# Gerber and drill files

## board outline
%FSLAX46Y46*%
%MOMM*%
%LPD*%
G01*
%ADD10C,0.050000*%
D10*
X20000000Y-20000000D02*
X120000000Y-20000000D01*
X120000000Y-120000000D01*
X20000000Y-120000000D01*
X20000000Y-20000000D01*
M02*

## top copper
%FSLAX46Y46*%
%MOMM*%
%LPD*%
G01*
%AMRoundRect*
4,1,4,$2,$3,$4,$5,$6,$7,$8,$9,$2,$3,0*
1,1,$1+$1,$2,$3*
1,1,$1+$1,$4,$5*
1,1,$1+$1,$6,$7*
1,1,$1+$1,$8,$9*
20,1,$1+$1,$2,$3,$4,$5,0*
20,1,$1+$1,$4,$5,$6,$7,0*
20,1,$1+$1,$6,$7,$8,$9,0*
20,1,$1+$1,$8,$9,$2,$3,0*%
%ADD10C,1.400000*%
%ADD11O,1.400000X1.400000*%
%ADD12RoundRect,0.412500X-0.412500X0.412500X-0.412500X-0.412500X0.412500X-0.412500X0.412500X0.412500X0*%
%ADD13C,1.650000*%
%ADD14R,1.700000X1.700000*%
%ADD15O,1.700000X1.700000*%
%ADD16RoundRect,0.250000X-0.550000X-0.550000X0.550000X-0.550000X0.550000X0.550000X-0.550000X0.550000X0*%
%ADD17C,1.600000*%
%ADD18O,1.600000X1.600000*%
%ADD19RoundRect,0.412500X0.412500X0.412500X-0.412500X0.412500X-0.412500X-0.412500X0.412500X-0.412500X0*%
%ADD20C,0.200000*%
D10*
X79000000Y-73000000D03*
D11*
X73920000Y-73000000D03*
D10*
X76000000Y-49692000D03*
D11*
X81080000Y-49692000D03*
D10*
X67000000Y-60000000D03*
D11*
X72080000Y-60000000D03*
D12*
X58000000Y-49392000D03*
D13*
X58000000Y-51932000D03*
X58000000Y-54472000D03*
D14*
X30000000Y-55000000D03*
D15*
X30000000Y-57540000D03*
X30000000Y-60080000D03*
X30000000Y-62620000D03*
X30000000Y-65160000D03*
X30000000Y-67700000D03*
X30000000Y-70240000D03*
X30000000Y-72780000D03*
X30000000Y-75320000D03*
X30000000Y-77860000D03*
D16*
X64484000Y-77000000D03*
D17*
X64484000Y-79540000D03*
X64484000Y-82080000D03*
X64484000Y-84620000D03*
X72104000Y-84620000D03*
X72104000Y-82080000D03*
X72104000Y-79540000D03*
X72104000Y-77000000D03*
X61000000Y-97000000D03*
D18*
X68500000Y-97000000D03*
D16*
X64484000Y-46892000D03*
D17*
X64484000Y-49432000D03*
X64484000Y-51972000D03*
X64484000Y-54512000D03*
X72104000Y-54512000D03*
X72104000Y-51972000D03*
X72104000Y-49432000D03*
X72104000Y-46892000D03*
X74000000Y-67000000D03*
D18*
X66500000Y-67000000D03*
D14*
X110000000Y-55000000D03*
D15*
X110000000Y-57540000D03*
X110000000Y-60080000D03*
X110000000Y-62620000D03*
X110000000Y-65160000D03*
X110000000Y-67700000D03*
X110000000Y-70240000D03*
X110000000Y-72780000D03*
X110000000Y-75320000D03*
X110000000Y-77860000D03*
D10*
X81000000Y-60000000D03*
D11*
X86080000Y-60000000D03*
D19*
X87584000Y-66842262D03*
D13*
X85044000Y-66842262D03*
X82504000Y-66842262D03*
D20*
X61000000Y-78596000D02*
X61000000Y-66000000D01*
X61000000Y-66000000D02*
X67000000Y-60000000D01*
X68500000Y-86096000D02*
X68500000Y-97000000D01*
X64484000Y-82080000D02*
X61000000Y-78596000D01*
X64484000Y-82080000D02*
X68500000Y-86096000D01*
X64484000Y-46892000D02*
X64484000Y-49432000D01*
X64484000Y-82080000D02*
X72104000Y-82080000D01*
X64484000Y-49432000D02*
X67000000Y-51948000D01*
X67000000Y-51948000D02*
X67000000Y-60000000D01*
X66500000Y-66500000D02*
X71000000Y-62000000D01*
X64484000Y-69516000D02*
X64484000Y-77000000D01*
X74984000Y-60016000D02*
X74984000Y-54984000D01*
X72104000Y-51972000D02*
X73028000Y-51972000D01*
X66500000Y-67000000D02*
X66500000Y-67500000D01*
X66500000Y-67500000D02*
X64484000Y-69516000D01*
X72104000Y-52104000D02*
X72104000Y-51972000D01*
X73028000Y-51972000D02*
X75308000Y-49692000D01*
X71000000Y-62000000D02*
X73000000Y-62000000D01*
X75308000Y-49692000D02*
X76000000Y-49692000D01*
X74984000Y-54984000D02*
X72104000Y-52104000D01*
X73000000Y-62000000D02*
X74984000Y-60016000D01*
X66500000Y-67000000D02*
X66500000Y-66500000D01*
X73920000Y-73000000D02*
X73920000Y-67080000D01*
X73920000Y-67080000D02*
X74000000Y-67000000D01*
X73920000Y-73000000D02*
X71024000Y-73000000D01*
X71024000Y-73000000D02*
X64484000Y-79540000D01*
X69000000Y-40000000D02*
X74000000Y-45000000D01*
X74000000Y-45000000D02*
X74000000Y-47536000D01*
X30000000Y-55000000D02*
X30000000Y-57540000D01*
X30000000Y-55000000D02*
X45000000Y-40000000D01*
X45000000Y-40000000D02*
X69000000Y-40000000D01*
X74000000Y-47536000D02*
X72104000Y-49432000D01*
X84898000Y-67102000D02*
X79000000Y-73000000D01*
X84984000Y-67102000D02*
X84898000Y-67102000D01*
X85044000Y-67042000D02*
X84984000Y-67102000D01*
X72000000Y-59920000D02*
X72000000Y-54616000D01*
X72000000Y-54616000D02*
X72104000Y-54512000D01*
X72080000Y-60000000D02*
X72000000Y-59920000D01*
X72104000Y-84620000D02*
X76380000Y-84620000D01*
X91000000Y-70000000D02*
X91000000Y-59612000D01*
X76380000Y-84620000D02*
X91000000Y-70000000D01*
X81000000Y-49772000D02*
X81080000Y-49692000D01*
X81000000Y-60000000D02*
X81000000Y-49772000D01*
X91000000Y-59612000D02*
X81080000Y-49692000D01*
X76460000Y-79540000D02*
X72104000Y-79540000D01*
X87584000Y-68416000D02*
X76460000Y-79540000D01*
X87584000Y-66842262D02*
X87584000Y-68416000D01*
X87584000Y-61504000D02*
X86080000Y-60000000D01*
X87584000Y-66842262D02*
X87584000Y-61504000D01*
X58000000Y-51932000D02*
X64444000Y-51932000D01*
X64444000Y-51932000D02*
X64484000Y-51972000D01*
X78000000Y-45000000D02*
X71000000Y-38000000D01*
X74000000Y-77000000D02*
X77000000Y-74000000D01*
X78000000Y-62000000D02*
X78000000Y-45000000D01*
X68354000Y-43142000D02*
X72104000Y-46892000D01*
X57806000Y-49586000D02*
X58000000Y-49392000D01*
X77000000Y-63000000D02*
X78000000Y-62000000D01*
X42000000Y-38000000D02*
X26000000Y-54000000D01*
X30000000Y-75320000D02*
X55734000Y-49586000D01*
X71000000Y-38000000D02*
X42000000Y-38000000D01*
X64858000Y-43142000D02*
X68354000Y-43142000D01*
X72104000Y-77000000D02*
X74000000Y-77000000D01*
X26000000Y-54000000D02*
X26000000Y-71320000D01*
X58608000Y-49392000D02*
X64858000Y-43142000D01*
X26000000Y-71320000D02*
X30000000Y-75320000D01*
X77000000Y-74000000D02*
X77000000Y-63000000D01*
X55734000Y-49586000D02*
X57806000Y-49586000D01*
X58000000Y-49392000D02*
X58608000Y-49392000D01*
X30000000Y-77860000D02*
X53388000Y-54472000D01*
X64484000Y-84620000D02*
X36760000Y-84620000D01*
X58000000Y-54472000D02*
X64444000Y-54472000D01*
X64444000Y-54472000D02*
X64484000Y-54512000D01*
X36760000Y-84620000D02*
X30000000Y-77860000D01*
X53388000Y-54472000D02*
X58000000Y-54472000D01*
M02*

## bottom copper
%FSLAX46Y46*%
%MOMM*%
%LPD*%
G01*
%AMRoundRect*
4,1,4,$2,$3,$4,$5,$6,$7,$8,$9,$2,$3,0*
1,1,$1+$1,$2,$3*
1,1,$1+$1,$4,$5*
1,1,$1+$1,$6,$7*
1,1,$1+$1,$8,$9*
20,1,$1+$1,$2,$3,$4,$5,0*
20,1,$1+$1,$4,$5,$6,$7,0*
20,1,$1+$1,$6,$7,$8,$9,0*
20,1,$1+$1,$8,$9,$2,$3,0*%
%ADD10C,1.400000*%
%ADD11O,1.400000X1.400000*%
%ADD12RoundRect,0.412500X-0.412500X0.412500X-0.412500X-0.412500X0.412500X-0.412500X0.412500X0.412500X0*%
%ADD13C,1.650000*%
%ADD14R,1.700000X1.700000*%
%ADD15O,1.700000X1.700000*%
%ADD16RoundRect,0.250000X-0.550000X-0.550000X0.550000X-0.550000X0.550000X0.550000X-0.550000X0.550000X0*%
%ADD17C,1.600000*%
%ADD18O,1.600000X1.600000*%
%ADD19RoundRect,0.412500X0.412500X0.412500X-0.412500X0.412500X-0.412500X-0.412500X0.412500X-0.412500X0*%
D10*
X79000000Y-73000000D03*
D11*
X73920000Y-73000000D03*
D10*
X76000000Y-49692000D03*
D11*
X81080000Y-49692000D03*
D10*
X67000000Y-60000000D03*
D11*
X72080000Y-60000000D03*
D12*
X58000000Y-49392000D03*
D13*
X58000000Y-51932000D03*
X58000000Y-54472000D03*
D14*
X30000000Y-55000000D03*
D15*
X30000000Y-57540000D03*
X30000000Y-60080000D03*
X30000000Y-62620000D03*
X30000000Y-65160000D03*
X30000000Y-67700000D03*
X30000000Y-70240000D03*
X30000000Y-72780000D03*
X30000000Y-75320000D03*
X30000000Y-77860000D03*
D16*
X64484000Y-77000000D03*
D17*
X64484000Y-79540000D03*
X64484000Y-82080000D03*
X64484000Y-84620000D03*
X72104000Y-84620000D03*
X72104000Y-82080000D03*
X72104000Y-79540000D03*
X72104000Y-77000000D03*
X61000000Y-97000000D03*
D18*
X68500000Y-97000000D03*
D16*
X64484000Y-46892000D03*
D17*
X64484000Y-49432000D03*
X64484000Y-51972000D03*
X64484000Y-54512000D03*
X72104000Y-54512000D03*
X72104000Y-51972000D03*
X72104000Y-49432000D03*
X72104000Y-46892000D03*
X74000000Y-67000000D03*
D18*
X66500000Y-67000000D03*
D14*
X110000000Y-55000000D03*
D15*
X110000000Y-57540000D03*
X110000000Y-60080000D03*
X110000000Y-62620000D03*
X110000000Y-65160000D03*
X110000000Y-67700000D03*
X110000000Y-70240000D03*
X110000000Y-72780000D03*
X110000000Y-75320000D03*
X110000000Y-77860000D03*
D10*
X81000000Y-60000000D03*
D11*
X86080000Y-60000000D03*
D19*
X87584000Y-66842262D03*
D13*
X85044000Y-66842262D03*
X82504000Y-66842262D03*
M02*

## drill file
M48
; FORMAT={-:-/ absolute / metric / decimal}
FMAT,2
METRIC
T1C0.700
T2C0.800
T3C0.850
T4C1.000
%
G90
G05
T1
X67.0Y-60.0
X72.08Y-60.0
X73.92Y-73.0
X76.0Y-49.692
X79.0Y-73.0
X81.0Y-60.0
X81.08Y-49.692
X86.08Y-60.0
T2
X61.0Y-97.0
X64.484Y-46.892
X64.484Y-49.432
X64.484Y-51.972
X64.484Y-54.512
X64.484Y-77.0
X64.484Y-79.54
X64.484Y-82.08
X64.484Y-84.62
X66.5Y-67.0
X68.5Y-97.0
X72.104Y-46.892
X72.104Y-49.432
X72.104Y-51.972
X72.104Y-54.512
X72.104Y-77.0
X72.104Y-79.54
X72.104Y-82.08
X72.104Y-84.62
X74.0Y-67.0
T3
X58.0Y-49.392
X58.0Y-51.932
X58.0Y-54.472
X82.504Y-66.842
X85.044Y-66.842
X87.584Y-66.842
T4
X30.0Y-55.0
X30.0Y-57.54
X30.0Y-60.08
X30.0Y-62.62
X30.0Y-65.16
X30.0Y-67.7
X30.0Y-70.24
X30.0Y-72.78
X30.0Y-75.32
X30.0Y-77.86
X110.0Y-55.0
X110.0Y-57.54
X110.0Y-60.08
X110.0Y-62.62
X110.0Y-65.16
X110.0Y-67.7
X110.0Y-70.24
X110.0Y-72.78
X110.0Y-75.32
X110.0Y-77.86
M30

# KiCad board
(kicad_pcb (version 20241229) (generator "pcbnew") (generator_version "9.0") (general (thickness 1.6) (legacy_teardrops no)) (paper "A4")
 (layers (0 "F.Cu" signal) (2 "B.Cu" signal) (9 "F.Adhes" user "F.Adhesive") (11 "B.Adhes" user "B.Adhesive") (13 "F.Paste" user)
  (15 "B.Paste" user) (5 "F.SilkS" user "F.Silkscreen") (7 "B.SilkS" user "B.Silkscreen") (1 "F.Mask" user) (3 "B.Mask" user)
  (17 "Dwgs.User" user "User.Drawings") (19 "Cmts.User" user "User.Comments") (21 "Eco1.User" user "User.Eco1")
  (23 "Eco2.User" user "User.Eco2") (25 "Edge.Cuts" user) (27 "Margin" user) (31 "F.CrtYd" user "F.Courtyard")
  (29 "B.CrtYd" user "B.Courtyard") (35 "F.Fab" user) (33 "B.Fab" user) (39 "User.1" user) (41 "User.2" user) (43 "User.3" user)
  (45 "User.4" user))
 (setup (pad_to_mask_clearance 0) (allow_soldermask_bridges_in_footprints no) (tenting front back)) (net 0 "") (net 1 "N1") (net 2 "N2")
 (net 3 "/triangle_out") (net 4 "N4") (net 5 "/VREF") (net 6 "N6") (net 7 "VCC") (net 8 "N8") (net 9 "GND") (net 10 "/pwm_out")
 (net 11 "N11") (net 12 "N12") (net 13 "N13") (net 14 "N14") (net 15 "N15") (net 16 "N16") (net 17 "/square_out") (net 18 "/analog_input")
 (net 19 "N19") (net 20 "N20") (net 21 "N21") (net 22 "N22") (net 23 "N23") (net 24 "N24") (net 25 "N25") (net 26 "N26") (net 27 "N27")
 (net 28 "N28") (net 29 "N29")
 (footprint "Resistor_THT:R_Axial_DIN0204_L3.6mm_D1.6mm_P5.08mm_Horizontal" (layer "F.Cu") (at 79 73 180)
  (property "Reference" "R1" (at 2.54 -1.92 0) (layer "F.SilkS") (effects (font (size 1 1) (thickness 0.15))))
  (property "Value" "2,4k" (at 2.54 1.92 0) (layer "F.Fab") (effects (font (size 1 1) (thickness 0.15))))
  (pad "1" thru_hole circle (at 0 0 180) (size 1.4 1.4) (drill 0.7) (layers "*.Cu" "*.Mask") (remove_unused_layers no) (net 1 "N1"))
  (pad "2" thru_hole oval (at 5.08 0 180) (size 1.4 1.4) (drill 0.7) (layers "*.Cu" "*.Mask") (remove_unused_layers no) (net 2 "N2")))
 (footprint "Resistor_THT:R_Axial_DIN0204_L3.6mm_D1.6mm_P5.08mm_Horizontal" (layer "F.Cu") (at 76 49.692)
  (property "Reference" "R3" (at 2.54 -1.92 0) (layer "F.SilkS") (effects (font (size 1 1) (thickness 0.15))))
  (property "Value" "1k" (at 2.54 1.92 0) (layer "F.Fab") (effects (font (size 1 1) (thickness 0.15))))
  (pad "1" thru_hole circle (at 0 0) (size 1.4 1.4) (drill 0.7) (layers "*.Cu" "*.Mask") (remove_unused_layers no) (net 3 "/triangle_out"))
  (pad "2" thru_hole oval (at 5.08 0) (size 1.4 1.4) (drill 0.7) (layers "*.Cu" "*.Mask") (remove_unused_layers no) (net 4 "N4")))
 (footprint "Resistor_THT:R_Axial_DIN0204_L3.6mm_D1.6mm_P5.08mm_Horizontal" (layer "F.Cu") (at 67 60)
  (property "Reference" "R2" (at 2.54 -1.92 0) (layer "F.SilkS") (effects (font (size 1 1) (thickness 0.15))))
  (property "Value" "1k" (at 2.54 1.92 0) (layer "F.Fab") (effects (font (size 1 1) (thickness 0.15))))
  (pad "1" thru_hole circle (at 0 0) (size 1.4 1.4) (drill 0.7) (layers "*.Cu" "*.Mask") (remove_unused_layers no) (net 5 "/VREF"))
  (pad "2" thru_hole oval (at 5.08 0) (size 1.4 1.4) (drill 0.7) (layers "*.Cu" "*.Mask") (remove_unused_layers no) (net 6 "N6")))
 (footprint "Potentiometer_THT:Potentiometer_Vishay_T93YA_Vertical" (layer "F.Cu") (at 58 49.392 -90)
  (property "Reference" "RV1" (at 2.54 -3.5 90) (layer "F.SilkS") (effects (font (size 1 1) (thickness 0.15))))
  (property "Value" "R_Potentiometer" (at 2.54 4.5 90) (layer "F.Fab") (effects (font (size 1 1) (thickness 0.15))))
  (pad "1" thru_hole roundrect (at 0 0 270) (size 1.65 1.65) (drill 0.85) (layers "*.Cu" "*.Mask") (remove_unused_layers no)
   (roundrect_rratio 0.25) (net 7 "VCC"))
  (pad "2" thru_hole circle (at 2.54 0 270) (size 1.65 1.65) (drill 0.85) (layers "*.Cu" "*.Mask") (remove_unused_layers no) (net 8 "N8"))
  (pad "3" thru_hole circle (at 5.08 0 270) (size 1.65 1.65) (drill 0.85) (layers "*.Cu" "*.Mask") (remove_unused_layers no) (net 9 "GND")))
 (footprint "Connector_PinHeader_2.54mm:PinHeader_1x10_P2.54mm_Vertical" (layer "F.Cu") (at 30 55)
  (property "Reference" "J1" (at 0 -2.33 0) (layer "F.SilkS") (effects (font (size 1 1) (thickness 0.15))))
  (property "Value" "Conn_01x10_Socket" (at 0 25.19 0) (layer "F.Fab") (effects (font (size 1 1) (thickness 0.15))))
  (pad "1" thru_hole rect (at 0 0) (size 1.7 1.7) (drill 1) (layers "*.Cu" "*.Mask") (remove_unused_layers no) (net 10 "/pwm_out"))
  (pad "2" thru_hole oval (at 0 2.54) (size 1.7 1.7) (drill 1) (layers "*.Cu" "*.Mask") (remove_unused_layers no) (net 10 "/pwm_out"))
  (pad "3" thru_hole oval (at 0 5.08) (size 1.7 1.7) (drill 1) (layers "*.Cu" "*.Mask") (remove_unused_layers no) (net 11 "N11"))
  (pad "4" thru_hole oval (at 0 7.62) (size 1.7 1.7) (drill 1) (layers "*.Cu" "*.Mask") (remove_unused_layers no) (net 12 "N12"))
  (pad "5" thru_hole oval (at 0 10.16) (size 1.7 1.7) (drill 1) (layers "*.Cu" "*.Mask") (remove_unused_layers no) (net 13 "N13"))
  (pad "6" thru_hole oval (at 0 12.7) (size 1.7 1.7) (drill 1) (layers "*.Cu" "*.Mask") (remove_unused_layers no) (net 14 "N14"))
  (pad "7" thru_hole oval (at 0 15.24) (size 1.7 1.7) (drill 1) (layers "*.Cu" "*.Mask") (remove_unused_layers no) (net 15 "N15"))
  (pad "8" thru_hole oval (at 0 17.78) (size 1.7 1.7) (drill 1) (layers "*.Cu" "*.Mask") (remove_unused_layers no) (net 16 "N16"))
  (pad "9" thru_hole oval (at 0 20.32) (size 1.7 1.7) (drill 1) (layers "*.Cu" "*.Mask") (remove_unused_layers no) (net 7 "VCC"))
  (pad "10" thru_hole oval (at 0 22.86) (size 1.7 1.7) (drill 1) (layers "*.Cu" "*.Mask") (remove_unused_layers no) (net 9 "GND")))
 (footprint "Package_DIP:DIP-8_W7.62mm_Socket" (layer "F.Cu") (at 64.484 77)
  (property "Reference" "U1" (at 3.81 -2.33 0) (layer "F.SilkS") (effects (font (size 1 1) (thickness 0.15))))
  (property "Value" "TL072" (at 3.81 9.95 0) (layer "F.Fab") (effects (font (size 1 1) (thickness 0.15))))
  (pad "1" thru_hole roundrect (at 0 0) (size 1.6 1.6) (drill 0.8) (layers "*.Cu" "*.Mask") (remove_unused_layers no)
   (roundrect_rratio 0.15625) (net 3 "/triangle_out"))
  (pad "2" thru_hole circle (at 0 2.54) (size 1.6 1.6) (drill 0.8) (layers "*.Cu" "*.Mask") (remove_unused_layers no) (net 2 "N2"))
  (pad "3" thru_hole circle (at 0 5.08) (size 1.6 1.6) (drill 0.8) (layers "*.Cu" "*.Mask") (remove_unused_layers no) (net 5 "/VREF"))
  (pad "4" thru_hole circle (at 0 7.62) (size 1.6 1.6) (drill 0.8) (layers "*.Cu" "*.Mask") (remove_unused_layers no) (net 9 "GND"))
  (pad "5" thru_hole circle (at 7.62 7.62) (size 1.6 1.6) (drill 0.8) (layers "*.Cu" "*.Mask") (remove_unused_layers no) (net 4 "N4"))
  (pad "6" thru_hole circle (at 7.62 5.08) (size 1.6 1.6) (drill 0.8) (layers "*.Cu" "*.Mask") (remove_unused_layers no) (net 5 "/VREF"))
  (pad "7" thru_hole circle (at 7.62 2.54) (size 1.6 1.6) (drill 0.8) (layers "*.Cu" "*.Mask") (remove_unused_layers no)
   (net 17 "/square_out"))
  (pad "8" thru_hole circle (at 7.62 0) (size 1.6 1.6) (drill 0.8) (layers "*.Cu" "*.Mask") (remove_unused_layers no) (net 7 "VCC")))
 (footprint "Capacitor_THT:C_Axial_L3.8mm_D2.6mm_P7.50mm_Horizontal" (layer "F.Cu") (at 61 97)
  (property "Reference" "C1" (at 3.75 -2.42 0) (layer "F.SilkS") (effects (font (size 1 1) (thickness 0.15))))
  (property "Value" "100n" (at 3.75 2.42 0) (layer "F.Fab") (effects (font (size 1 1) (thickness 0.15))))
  (pad "1" thru_hole circle (at 0 0) (size 1.6 1.6) (drill 0.8) (layers "*.Cu" "*.Mask") (remove_unused_layers no) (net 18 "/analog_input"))
  (pad "2" thru_hole oval (at 7.5 0) (size 1.6 1.6) (drill 0.8) (layers "*.Cu" "*.Mask") (remove_unused_layers no) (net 5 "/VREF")))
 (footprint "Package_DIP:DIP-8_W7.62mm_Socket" (layer "F.Cu") (at 64.484 46.892)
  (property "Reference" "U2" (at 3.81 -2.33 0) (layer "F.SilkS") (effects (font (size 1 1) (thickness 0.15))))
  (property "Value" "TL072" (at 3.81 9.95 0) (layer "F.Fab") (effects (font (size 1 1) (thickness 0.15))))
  (pad "1" thru_hole roundrect (at 0 0) (size 1.6 1.6) (drill 0.8) (layers "*.Cu" "*.Mask") (remove_unused_layers no)
   (roundrect_rratio 0.15625) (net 5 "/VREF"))
  (pad "2" thru_hole circle (at 0 2.54) (size 1.6 1.6) (drill 0.8) (layers "*.Cu" "*.Mask") (remove_unused_layers no) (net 5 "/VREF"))
  (pad "3" thru_hole circle (at 0 5.08) (size 1.6 1.6) (drill 0.8) (layers "*.Cu" "*.Mask") (remove_unused_layers no) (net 8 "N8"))
  (pad "4" thru_hole circle (at 0 7.62) (size 1.6 1.6) (drill 0.8) (layers "*.Cu" "*.Mask") (remove_unused_layers no) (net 9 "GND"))
  (pad "5" thru_hole circle (at 7.62 7.62) (size 1.6 1.6) (drill 0.8) (layers "*.Cu" "*.Mask") (remove_unused_layers no) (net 6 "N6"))
  (pad "6" thru_hole circle (at 7.62 5.08) (size 1.6 1.6) (drill 0.8) (layers "*.Cu" "*.Mask") (remove_unused_layers no)
   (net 3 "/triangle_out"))
  (pad "7" thru_hole circle (at 7.62 2.54) (size 1.6 1.6) (drill 0.8) (layers "*.Cu" "*.Mask") (remove_unused_layers no) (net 10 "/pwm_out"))
  (pad "8" thru_hole circle (at 7.62 0) (size 1.6 1.6) (drill 0.8) (layers "*.Cu" "*.Mask") (remove_unused_layers no) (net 7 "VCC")))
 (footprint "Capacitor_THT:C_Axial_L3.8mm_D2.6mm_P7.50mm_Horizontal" (layer "F.Cu") (at 74 67 180)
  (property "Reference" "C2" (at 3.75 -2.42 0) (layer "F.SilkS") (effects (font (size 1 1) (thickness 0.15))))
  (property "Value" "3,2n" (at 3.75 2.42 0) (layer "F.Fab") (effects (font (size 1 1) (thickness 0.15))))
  (pad "1" thru_hole circle (at 0 0 180) (size 1.6 1.6) (drill 0.8) (layers "*.Cu" "*.Mask") (remove_unused_layers no) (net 2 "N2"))
  (pad "2" thru_hole oval (at 7.5 0 180) (size 1.6 1.6) (drill 0.8) (layers "*.Cu" "*.Mask") (remove_unused_layers no)
   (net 3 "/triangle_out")))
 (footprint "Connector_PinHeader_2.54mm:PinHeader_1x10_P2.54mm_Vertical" (layer "F.Cu") (at 110 55)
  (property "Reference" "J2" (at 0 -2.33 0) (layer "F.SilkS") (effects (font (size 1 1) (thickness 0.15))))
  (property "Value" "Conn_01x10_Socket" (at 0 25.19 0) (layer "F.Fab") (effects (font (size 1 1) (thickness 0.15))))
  (pad "1" thru_hole rect (at 0 0) (size 1.7 1.7) (drill 1) (layers "*.Cu" "*.Mask") (remove_unused_layers no) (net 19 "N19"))
  (pad "2" thru_hole oval (at 0 2.54) (size 1.7 1.7) (drill 1) (layers "*.Cu" "*.Mask") (remove_unused_layers no) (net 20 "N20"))
  (pad "3" thru_hole oval (at 0 5.08) (size 1.7 1.7) (drill 1) (layers "*.Cu" "*.Mask") (remove_unused_layers no) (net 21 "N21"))
  (pad "4" thru_hole oval (at 0 7.62) (size 1.7 1.7) (drill 1) (layers "*.Cu" "*.Mask") (remove_unused_layers no) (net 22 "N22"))
  (pad "5" thru_hole oval (at 0 10.16) (size 1.7 1.7) (drill 1) (layers "*.Cu" "*.Mask") (remove_unused_layers no) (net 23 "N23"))
  (pad "6" thru_hole oval (at 0 12.7) (size 1.7 1.7) (drill 1) (layers "*.Cu" "*.Mask") (remove_unused_layers no) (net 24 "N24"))
  (pad "7" thru_hole oval (at 0 15.24) (size 1.7 1.7) (drill 1) (layers "*.Cu" "*.Mask") (remove_unused_layers no) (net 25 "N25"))
  (pad "8" thru_hole oval (at 0 17.78) (size 1.7 1.7) (drill 1) (layers "*.Cu" "*.Mask") (remove_unused_layers no) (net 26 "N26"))
  (pad "9" thru_hole oval (at 0 20.32) (size 1.7 1.7) (drill 1) (layers "*.Cu" "*.Mask") (remove_unused_layers no) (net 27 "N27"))
  (pad "10" thru_hole oval (at 0 22.86) (size 1.7 1.7) (drill 1) (layers "*.Cu" "*.Mask") (remove_unused_layers no) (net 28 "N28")))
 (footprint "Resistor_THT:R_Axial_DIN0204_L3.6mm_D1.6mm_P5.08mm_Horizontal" (layer "F.Cu") (at 81 60)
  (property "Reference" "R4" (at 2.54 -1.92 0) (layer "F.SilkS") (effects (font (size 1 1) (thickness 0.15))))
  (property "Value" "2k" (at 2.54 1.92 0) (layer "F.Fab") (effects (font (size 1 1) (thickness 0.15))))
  (pad "1" thru_hole circle (at 0 0) (size 1.4 1.4) (drill 0.7) (layers "*.Cu" "*.Mask") (remove_unused_layers no) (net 4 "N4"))
  (pad "2" thru_hole oval (at 5.08 0) (size 1.4 1.4) (drill 0.7) (layers "*.Cu" "*.Mask") (remove_unused_layers no) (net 17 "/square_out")))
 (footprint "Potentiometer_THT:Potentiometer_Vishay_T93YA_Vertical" (layer "F.Cu") (at 87.584 66.842262 180)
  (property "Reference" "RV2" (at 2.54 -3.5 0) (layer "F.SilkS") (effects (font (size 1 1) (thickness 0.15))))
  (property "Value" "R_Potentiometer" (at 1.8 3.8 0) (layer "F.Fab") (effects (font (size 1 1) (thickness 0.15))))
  (pad "1" thru_hole roundrect (at 0 0 180) (size 1.65 1.65) (drill 0.85) (layers "*.Cu" "*.Mask") (remove_unused_layers no)
   (roundrect_rratio 0.25) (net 17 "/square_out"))
  (pad "2" thru_hole circle (at 2.54 0 180) (size 1.65 1.65) (drill 0.85) (layers "*.Cu" "*.Mask") (remove_unused_layers no) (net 1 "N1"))
  (pad "3" thru_hole circle (at 5.08 0 180) (size 1.65 1.65) (drill 0.85) (layers "*.Cu" "*.Mask") (remove_unused_layers no) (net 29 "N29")))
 (gr_rect (start 20 20) (end 120 120) (stroke (width 0.05) (type default)) (fill no) (layer "Edge.Cuts"))
 (segment (start 61 78.596) (end 61 66) (width 0.2) (layer "F.Cu") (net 5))
 (segment (start 61 66) (end 67 60) (width 0.2) (layer "F.Cu") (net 5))
 (segment (start 68.5 86.096) (end 68.5 97) (width 0.2) (layer "F.Cu") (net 5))
 (segment (start 64.484 82.08) (end 61 78.596) (width 0.2) (layer "F.Cu") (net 5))
 (segment (start 64.484 82.08) (end 68.5 86.096) (width 0.2) (layer "F.Cu") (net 5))
 (segment (start 64.484 46.892) (end 64.484 49.432) (width 0.2) (layer "F.Cu") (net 5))
 (segment (start 64.484 82.08) (end 72.104 82.08) (width 0.2) (layer "F.Cu") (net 5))
 (segment (start 64.484 49.432) (end 67 51.948) (width 0.2) (layer "F.Cu") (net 5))
 (segment (start 67 51.948) (end 67 60) (width 0.2) (layer "F.Cu") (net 5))
 (segment (start 66.5 66.5) (end 71 62) (width 0.2) (layer "F.Cu") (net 3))
 (segment (start 64.484 69.516) (end 64.484 77) (width 0.2) (layer "F.Cu") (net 3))
 (segment (start 74.984 60.016) (end 74.984 54.984) (width 0.2) (layer "F.Cu") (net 3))
 (segment (start 72.104 51.972) (end 73.028 51.972) (width 0.2) (layer "F.Cu") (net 3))
 (segment (start 66.5 67) (end 66.5 67.5) (width 0.2) (layer "F.Cu") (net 3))
 (segment (start 66.5 67.5) (end 64.484 69.516) (width 0.2) (layer "F.Cu") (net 3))
 (segment (start 72.104 52.104) (end 72.104 51.972) (width 0.2) (layer "F.Cu") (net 3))
 (segment (start 73.028 51.972) (end 75.308 49.692) (width 0.2) (layer "F.Cu") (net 3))
 (segment (start 71 62) (end 73 62) (width 0.2) (layer "F.Cu") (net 3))
 (segment (start 75.308 49.692) (end 76 49.692) (width 0.2) (layer "F.Cu") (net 3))
 (segment (start 74.984 54.984) (end 72.104 52.104) (width 0.2) (layer "F.Cu") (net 3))
 (segment (start 73 62) (end 74.984 60.016) (width 0.2) (layer "F.Cu") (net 3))
 (segment (start 66.5 67) (end 66.5 66.5) (width 0.2) (layer "F.Cu") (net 3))
 (segment (start 73.92 73) (end 73.92 67.08) (width 0.2) (layer "F.Cu") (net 2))
 (segment (start 73.92 67.08) (end 74 67) (width 0.2) (layer "F.Cu") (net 2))
 (segment (start 73.92 73) (end 71.024 73) (width 0.2) (layer "F.Cu") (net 2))
 (segment (start 71.024 73) (end 64.484 79.54) (width 0.2) (layer "F.Cu") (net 2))
 (segment (start 69 40) (end 74 45) (width 0.2) (layer "F.Cu") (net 10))
 (segment (start 74 45) (end 74 47.536) (width 0.2) (layer "F.Cu") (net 10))
 (segment (start 30 55) (end 30 57.54) (width 0.2) (layer "F.Cu") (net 10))
 (segment (start 30 55) (end 45 40) (width 0.2) (layer "F.Cu") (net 10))
 (segment (start 45 40) (end 69 40) (width 0.2) (layer "F.Cu") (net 10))
 (segment (start 74 47.536) (end 72.104 49.432) (width 0.2) (layer "F.Cu") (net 10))
 (segment (start 84.898 67.102) (end 79 73) (width 0.2) (layer "F.Cu") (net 1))
 (segment (start 84.984 67.102) (end 84.898 67.102) (width 0.2) (layer "F.Cu") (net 1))
 (segment (start 85.044 67.042) (end 84.984 67.102) (width 0.2) (layer "F.Cu") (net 1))
 (segment (start 72 59.92) (end 72 54.616) (width 0.2) (layer "F.Cu") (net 6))
 (segment (start 72 54.616) (end 72.104 54.512) (width 0.2) (layer "F.Cu") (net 6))
 (segment (start 72.08 60) (end 72 59.92) (width 0.2) (layer "F.Cu") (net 6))
 (segment (start 72.104 84.62) (end 76.38 84.62) (width 0.2) (layer "F.Cu") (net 4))
 (segment (start 91 70) (end 91 59.612) (width 0.2) (layer "F.Cu") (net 4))
 (segment (start 76.38 84.62) (end 91 70) (width 0.2) (layer "F.Cu") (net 4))
 (segment (start 81 49.772) (end 81.08 49.692) (width 0.2) (layer "F.Cu") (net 4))
 (segment (start 81 60) (end 81 49.772) (width 0.2) (layer "F.Cu") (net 4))
 (segment (start 91 59.612) (end 81.08 49.692) (width 0.2) (layer "F.Cu") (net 4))
 (segment (start 76.46 79.54) (end 72.104 79.54) (width 0.2) (layer "F.Cu") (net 17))
 (segment (start 87.584 68.416) (end 76.46 79.54) (width 0.2) (layer "F.Cu") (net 17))
 (segment (start 87.584 66.842262) (end 87.584 68.416) (width 0.2) (layer "F.Cu") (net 17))
 (segment (start 87.584 61.504) (end 86.08 60) (width 0.2) (layer "F.Cu") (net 17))
 (segment (start 87.584 66.842262) (end 87.584 61.504) (width 0.2) (layer "F.Cu") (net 17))
 (segment (start 58 51.932) (end 64.444 51.932) (width 0.2) (layer "F.Cu") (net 8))
 (segment (start 64.444 51.932) (end 64.484 51.972) (width 0.2) (layer "F.Cu") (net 8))
 (segment (start 78 45) (end 71 38) (width 0.2) (layer "F.Cu") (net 7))
 (segment (start 74 77) (end 77 74) (width 0.2) (layer "F.Cu") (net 7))
 (segment (start 78 62) (end 78 45) (width 0.2) (layer "F.Cu") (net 7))
 (segment (start 68.354 43.142) (end 72.104 46.892) (width 0.2) (layer "F.Cu") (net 7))
 (segment (start 57.806 49.586) (end 58 49.392) (width 0.2) (layer "F.Cu") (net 7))
 (segment (start 77 63) (end 78 62) (width 0.2) (layer "F.Cu") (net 7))
 (segment (start 42 38) (end 26 54) (width 0.2) (layer "F.Cu") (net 7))
 (segment (start 30 75.32) (end 55.734 49.586) (width 0.2) (layer "F.Cu") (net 7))
 (segment (start 71 38) (end 42 38) (width 0.2) (layer "F.Cu") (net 7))
 (segment (start 64.858 43.142) (end 68.354 43.142) (width 0.2) (layer "F.Cu") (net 7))
 (segment (start 72.104 77) (end 74 77) (width 0.2) (layer "F.Cu") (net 7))
 (segment (start 26 54) (end 26 71.32) (width 0.2) (layer "F.Cu") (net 7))
 (segment (start 58.608 49.392) (end 64.858 43.142) (width 0.2) (layer "F.Cu") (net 7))
 (segment (start 26 71.32) (end 30 75.32) (width 0.2) (layer "F.Cu") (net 7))
 (segment (start 77 74) (end 77 63) (width 0.2) (layer "F.Cu") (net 7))
 (segment (start 55.734 49.586) (end 57.806 49.586) (width 0.2) (layer "F.Cu") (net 7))
 (segment (start 58 49.392) (end 58.608 49.392) (width 0.2) (layer "F.Cu") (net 7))
 (segment (start 30 77.86) (end 53.388 54.472) (width 0.2) (layer "F.Cu") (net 9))
 (segment (start 64.484 84.62) (end 36.76 84.62) (width 0.2) (layer "F.Cu") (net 9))
 (segment (start 58 54.472) (end 64.444 54.472) (width 0.2) (layer "F.Cu") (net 9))
 (segment (start 64.444 54.472) (end 64.484 54.512) (width 0.2) (layer "F.Cu") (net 9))
 (segment (start 36.76 84.62) (end 30 77.86) (width 0.2) (layer "F.Cu") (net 9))
 (segment (start 53.388 54.472) (end 58 54.472) (width 0.2) (layer "F.Cu") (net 9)))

